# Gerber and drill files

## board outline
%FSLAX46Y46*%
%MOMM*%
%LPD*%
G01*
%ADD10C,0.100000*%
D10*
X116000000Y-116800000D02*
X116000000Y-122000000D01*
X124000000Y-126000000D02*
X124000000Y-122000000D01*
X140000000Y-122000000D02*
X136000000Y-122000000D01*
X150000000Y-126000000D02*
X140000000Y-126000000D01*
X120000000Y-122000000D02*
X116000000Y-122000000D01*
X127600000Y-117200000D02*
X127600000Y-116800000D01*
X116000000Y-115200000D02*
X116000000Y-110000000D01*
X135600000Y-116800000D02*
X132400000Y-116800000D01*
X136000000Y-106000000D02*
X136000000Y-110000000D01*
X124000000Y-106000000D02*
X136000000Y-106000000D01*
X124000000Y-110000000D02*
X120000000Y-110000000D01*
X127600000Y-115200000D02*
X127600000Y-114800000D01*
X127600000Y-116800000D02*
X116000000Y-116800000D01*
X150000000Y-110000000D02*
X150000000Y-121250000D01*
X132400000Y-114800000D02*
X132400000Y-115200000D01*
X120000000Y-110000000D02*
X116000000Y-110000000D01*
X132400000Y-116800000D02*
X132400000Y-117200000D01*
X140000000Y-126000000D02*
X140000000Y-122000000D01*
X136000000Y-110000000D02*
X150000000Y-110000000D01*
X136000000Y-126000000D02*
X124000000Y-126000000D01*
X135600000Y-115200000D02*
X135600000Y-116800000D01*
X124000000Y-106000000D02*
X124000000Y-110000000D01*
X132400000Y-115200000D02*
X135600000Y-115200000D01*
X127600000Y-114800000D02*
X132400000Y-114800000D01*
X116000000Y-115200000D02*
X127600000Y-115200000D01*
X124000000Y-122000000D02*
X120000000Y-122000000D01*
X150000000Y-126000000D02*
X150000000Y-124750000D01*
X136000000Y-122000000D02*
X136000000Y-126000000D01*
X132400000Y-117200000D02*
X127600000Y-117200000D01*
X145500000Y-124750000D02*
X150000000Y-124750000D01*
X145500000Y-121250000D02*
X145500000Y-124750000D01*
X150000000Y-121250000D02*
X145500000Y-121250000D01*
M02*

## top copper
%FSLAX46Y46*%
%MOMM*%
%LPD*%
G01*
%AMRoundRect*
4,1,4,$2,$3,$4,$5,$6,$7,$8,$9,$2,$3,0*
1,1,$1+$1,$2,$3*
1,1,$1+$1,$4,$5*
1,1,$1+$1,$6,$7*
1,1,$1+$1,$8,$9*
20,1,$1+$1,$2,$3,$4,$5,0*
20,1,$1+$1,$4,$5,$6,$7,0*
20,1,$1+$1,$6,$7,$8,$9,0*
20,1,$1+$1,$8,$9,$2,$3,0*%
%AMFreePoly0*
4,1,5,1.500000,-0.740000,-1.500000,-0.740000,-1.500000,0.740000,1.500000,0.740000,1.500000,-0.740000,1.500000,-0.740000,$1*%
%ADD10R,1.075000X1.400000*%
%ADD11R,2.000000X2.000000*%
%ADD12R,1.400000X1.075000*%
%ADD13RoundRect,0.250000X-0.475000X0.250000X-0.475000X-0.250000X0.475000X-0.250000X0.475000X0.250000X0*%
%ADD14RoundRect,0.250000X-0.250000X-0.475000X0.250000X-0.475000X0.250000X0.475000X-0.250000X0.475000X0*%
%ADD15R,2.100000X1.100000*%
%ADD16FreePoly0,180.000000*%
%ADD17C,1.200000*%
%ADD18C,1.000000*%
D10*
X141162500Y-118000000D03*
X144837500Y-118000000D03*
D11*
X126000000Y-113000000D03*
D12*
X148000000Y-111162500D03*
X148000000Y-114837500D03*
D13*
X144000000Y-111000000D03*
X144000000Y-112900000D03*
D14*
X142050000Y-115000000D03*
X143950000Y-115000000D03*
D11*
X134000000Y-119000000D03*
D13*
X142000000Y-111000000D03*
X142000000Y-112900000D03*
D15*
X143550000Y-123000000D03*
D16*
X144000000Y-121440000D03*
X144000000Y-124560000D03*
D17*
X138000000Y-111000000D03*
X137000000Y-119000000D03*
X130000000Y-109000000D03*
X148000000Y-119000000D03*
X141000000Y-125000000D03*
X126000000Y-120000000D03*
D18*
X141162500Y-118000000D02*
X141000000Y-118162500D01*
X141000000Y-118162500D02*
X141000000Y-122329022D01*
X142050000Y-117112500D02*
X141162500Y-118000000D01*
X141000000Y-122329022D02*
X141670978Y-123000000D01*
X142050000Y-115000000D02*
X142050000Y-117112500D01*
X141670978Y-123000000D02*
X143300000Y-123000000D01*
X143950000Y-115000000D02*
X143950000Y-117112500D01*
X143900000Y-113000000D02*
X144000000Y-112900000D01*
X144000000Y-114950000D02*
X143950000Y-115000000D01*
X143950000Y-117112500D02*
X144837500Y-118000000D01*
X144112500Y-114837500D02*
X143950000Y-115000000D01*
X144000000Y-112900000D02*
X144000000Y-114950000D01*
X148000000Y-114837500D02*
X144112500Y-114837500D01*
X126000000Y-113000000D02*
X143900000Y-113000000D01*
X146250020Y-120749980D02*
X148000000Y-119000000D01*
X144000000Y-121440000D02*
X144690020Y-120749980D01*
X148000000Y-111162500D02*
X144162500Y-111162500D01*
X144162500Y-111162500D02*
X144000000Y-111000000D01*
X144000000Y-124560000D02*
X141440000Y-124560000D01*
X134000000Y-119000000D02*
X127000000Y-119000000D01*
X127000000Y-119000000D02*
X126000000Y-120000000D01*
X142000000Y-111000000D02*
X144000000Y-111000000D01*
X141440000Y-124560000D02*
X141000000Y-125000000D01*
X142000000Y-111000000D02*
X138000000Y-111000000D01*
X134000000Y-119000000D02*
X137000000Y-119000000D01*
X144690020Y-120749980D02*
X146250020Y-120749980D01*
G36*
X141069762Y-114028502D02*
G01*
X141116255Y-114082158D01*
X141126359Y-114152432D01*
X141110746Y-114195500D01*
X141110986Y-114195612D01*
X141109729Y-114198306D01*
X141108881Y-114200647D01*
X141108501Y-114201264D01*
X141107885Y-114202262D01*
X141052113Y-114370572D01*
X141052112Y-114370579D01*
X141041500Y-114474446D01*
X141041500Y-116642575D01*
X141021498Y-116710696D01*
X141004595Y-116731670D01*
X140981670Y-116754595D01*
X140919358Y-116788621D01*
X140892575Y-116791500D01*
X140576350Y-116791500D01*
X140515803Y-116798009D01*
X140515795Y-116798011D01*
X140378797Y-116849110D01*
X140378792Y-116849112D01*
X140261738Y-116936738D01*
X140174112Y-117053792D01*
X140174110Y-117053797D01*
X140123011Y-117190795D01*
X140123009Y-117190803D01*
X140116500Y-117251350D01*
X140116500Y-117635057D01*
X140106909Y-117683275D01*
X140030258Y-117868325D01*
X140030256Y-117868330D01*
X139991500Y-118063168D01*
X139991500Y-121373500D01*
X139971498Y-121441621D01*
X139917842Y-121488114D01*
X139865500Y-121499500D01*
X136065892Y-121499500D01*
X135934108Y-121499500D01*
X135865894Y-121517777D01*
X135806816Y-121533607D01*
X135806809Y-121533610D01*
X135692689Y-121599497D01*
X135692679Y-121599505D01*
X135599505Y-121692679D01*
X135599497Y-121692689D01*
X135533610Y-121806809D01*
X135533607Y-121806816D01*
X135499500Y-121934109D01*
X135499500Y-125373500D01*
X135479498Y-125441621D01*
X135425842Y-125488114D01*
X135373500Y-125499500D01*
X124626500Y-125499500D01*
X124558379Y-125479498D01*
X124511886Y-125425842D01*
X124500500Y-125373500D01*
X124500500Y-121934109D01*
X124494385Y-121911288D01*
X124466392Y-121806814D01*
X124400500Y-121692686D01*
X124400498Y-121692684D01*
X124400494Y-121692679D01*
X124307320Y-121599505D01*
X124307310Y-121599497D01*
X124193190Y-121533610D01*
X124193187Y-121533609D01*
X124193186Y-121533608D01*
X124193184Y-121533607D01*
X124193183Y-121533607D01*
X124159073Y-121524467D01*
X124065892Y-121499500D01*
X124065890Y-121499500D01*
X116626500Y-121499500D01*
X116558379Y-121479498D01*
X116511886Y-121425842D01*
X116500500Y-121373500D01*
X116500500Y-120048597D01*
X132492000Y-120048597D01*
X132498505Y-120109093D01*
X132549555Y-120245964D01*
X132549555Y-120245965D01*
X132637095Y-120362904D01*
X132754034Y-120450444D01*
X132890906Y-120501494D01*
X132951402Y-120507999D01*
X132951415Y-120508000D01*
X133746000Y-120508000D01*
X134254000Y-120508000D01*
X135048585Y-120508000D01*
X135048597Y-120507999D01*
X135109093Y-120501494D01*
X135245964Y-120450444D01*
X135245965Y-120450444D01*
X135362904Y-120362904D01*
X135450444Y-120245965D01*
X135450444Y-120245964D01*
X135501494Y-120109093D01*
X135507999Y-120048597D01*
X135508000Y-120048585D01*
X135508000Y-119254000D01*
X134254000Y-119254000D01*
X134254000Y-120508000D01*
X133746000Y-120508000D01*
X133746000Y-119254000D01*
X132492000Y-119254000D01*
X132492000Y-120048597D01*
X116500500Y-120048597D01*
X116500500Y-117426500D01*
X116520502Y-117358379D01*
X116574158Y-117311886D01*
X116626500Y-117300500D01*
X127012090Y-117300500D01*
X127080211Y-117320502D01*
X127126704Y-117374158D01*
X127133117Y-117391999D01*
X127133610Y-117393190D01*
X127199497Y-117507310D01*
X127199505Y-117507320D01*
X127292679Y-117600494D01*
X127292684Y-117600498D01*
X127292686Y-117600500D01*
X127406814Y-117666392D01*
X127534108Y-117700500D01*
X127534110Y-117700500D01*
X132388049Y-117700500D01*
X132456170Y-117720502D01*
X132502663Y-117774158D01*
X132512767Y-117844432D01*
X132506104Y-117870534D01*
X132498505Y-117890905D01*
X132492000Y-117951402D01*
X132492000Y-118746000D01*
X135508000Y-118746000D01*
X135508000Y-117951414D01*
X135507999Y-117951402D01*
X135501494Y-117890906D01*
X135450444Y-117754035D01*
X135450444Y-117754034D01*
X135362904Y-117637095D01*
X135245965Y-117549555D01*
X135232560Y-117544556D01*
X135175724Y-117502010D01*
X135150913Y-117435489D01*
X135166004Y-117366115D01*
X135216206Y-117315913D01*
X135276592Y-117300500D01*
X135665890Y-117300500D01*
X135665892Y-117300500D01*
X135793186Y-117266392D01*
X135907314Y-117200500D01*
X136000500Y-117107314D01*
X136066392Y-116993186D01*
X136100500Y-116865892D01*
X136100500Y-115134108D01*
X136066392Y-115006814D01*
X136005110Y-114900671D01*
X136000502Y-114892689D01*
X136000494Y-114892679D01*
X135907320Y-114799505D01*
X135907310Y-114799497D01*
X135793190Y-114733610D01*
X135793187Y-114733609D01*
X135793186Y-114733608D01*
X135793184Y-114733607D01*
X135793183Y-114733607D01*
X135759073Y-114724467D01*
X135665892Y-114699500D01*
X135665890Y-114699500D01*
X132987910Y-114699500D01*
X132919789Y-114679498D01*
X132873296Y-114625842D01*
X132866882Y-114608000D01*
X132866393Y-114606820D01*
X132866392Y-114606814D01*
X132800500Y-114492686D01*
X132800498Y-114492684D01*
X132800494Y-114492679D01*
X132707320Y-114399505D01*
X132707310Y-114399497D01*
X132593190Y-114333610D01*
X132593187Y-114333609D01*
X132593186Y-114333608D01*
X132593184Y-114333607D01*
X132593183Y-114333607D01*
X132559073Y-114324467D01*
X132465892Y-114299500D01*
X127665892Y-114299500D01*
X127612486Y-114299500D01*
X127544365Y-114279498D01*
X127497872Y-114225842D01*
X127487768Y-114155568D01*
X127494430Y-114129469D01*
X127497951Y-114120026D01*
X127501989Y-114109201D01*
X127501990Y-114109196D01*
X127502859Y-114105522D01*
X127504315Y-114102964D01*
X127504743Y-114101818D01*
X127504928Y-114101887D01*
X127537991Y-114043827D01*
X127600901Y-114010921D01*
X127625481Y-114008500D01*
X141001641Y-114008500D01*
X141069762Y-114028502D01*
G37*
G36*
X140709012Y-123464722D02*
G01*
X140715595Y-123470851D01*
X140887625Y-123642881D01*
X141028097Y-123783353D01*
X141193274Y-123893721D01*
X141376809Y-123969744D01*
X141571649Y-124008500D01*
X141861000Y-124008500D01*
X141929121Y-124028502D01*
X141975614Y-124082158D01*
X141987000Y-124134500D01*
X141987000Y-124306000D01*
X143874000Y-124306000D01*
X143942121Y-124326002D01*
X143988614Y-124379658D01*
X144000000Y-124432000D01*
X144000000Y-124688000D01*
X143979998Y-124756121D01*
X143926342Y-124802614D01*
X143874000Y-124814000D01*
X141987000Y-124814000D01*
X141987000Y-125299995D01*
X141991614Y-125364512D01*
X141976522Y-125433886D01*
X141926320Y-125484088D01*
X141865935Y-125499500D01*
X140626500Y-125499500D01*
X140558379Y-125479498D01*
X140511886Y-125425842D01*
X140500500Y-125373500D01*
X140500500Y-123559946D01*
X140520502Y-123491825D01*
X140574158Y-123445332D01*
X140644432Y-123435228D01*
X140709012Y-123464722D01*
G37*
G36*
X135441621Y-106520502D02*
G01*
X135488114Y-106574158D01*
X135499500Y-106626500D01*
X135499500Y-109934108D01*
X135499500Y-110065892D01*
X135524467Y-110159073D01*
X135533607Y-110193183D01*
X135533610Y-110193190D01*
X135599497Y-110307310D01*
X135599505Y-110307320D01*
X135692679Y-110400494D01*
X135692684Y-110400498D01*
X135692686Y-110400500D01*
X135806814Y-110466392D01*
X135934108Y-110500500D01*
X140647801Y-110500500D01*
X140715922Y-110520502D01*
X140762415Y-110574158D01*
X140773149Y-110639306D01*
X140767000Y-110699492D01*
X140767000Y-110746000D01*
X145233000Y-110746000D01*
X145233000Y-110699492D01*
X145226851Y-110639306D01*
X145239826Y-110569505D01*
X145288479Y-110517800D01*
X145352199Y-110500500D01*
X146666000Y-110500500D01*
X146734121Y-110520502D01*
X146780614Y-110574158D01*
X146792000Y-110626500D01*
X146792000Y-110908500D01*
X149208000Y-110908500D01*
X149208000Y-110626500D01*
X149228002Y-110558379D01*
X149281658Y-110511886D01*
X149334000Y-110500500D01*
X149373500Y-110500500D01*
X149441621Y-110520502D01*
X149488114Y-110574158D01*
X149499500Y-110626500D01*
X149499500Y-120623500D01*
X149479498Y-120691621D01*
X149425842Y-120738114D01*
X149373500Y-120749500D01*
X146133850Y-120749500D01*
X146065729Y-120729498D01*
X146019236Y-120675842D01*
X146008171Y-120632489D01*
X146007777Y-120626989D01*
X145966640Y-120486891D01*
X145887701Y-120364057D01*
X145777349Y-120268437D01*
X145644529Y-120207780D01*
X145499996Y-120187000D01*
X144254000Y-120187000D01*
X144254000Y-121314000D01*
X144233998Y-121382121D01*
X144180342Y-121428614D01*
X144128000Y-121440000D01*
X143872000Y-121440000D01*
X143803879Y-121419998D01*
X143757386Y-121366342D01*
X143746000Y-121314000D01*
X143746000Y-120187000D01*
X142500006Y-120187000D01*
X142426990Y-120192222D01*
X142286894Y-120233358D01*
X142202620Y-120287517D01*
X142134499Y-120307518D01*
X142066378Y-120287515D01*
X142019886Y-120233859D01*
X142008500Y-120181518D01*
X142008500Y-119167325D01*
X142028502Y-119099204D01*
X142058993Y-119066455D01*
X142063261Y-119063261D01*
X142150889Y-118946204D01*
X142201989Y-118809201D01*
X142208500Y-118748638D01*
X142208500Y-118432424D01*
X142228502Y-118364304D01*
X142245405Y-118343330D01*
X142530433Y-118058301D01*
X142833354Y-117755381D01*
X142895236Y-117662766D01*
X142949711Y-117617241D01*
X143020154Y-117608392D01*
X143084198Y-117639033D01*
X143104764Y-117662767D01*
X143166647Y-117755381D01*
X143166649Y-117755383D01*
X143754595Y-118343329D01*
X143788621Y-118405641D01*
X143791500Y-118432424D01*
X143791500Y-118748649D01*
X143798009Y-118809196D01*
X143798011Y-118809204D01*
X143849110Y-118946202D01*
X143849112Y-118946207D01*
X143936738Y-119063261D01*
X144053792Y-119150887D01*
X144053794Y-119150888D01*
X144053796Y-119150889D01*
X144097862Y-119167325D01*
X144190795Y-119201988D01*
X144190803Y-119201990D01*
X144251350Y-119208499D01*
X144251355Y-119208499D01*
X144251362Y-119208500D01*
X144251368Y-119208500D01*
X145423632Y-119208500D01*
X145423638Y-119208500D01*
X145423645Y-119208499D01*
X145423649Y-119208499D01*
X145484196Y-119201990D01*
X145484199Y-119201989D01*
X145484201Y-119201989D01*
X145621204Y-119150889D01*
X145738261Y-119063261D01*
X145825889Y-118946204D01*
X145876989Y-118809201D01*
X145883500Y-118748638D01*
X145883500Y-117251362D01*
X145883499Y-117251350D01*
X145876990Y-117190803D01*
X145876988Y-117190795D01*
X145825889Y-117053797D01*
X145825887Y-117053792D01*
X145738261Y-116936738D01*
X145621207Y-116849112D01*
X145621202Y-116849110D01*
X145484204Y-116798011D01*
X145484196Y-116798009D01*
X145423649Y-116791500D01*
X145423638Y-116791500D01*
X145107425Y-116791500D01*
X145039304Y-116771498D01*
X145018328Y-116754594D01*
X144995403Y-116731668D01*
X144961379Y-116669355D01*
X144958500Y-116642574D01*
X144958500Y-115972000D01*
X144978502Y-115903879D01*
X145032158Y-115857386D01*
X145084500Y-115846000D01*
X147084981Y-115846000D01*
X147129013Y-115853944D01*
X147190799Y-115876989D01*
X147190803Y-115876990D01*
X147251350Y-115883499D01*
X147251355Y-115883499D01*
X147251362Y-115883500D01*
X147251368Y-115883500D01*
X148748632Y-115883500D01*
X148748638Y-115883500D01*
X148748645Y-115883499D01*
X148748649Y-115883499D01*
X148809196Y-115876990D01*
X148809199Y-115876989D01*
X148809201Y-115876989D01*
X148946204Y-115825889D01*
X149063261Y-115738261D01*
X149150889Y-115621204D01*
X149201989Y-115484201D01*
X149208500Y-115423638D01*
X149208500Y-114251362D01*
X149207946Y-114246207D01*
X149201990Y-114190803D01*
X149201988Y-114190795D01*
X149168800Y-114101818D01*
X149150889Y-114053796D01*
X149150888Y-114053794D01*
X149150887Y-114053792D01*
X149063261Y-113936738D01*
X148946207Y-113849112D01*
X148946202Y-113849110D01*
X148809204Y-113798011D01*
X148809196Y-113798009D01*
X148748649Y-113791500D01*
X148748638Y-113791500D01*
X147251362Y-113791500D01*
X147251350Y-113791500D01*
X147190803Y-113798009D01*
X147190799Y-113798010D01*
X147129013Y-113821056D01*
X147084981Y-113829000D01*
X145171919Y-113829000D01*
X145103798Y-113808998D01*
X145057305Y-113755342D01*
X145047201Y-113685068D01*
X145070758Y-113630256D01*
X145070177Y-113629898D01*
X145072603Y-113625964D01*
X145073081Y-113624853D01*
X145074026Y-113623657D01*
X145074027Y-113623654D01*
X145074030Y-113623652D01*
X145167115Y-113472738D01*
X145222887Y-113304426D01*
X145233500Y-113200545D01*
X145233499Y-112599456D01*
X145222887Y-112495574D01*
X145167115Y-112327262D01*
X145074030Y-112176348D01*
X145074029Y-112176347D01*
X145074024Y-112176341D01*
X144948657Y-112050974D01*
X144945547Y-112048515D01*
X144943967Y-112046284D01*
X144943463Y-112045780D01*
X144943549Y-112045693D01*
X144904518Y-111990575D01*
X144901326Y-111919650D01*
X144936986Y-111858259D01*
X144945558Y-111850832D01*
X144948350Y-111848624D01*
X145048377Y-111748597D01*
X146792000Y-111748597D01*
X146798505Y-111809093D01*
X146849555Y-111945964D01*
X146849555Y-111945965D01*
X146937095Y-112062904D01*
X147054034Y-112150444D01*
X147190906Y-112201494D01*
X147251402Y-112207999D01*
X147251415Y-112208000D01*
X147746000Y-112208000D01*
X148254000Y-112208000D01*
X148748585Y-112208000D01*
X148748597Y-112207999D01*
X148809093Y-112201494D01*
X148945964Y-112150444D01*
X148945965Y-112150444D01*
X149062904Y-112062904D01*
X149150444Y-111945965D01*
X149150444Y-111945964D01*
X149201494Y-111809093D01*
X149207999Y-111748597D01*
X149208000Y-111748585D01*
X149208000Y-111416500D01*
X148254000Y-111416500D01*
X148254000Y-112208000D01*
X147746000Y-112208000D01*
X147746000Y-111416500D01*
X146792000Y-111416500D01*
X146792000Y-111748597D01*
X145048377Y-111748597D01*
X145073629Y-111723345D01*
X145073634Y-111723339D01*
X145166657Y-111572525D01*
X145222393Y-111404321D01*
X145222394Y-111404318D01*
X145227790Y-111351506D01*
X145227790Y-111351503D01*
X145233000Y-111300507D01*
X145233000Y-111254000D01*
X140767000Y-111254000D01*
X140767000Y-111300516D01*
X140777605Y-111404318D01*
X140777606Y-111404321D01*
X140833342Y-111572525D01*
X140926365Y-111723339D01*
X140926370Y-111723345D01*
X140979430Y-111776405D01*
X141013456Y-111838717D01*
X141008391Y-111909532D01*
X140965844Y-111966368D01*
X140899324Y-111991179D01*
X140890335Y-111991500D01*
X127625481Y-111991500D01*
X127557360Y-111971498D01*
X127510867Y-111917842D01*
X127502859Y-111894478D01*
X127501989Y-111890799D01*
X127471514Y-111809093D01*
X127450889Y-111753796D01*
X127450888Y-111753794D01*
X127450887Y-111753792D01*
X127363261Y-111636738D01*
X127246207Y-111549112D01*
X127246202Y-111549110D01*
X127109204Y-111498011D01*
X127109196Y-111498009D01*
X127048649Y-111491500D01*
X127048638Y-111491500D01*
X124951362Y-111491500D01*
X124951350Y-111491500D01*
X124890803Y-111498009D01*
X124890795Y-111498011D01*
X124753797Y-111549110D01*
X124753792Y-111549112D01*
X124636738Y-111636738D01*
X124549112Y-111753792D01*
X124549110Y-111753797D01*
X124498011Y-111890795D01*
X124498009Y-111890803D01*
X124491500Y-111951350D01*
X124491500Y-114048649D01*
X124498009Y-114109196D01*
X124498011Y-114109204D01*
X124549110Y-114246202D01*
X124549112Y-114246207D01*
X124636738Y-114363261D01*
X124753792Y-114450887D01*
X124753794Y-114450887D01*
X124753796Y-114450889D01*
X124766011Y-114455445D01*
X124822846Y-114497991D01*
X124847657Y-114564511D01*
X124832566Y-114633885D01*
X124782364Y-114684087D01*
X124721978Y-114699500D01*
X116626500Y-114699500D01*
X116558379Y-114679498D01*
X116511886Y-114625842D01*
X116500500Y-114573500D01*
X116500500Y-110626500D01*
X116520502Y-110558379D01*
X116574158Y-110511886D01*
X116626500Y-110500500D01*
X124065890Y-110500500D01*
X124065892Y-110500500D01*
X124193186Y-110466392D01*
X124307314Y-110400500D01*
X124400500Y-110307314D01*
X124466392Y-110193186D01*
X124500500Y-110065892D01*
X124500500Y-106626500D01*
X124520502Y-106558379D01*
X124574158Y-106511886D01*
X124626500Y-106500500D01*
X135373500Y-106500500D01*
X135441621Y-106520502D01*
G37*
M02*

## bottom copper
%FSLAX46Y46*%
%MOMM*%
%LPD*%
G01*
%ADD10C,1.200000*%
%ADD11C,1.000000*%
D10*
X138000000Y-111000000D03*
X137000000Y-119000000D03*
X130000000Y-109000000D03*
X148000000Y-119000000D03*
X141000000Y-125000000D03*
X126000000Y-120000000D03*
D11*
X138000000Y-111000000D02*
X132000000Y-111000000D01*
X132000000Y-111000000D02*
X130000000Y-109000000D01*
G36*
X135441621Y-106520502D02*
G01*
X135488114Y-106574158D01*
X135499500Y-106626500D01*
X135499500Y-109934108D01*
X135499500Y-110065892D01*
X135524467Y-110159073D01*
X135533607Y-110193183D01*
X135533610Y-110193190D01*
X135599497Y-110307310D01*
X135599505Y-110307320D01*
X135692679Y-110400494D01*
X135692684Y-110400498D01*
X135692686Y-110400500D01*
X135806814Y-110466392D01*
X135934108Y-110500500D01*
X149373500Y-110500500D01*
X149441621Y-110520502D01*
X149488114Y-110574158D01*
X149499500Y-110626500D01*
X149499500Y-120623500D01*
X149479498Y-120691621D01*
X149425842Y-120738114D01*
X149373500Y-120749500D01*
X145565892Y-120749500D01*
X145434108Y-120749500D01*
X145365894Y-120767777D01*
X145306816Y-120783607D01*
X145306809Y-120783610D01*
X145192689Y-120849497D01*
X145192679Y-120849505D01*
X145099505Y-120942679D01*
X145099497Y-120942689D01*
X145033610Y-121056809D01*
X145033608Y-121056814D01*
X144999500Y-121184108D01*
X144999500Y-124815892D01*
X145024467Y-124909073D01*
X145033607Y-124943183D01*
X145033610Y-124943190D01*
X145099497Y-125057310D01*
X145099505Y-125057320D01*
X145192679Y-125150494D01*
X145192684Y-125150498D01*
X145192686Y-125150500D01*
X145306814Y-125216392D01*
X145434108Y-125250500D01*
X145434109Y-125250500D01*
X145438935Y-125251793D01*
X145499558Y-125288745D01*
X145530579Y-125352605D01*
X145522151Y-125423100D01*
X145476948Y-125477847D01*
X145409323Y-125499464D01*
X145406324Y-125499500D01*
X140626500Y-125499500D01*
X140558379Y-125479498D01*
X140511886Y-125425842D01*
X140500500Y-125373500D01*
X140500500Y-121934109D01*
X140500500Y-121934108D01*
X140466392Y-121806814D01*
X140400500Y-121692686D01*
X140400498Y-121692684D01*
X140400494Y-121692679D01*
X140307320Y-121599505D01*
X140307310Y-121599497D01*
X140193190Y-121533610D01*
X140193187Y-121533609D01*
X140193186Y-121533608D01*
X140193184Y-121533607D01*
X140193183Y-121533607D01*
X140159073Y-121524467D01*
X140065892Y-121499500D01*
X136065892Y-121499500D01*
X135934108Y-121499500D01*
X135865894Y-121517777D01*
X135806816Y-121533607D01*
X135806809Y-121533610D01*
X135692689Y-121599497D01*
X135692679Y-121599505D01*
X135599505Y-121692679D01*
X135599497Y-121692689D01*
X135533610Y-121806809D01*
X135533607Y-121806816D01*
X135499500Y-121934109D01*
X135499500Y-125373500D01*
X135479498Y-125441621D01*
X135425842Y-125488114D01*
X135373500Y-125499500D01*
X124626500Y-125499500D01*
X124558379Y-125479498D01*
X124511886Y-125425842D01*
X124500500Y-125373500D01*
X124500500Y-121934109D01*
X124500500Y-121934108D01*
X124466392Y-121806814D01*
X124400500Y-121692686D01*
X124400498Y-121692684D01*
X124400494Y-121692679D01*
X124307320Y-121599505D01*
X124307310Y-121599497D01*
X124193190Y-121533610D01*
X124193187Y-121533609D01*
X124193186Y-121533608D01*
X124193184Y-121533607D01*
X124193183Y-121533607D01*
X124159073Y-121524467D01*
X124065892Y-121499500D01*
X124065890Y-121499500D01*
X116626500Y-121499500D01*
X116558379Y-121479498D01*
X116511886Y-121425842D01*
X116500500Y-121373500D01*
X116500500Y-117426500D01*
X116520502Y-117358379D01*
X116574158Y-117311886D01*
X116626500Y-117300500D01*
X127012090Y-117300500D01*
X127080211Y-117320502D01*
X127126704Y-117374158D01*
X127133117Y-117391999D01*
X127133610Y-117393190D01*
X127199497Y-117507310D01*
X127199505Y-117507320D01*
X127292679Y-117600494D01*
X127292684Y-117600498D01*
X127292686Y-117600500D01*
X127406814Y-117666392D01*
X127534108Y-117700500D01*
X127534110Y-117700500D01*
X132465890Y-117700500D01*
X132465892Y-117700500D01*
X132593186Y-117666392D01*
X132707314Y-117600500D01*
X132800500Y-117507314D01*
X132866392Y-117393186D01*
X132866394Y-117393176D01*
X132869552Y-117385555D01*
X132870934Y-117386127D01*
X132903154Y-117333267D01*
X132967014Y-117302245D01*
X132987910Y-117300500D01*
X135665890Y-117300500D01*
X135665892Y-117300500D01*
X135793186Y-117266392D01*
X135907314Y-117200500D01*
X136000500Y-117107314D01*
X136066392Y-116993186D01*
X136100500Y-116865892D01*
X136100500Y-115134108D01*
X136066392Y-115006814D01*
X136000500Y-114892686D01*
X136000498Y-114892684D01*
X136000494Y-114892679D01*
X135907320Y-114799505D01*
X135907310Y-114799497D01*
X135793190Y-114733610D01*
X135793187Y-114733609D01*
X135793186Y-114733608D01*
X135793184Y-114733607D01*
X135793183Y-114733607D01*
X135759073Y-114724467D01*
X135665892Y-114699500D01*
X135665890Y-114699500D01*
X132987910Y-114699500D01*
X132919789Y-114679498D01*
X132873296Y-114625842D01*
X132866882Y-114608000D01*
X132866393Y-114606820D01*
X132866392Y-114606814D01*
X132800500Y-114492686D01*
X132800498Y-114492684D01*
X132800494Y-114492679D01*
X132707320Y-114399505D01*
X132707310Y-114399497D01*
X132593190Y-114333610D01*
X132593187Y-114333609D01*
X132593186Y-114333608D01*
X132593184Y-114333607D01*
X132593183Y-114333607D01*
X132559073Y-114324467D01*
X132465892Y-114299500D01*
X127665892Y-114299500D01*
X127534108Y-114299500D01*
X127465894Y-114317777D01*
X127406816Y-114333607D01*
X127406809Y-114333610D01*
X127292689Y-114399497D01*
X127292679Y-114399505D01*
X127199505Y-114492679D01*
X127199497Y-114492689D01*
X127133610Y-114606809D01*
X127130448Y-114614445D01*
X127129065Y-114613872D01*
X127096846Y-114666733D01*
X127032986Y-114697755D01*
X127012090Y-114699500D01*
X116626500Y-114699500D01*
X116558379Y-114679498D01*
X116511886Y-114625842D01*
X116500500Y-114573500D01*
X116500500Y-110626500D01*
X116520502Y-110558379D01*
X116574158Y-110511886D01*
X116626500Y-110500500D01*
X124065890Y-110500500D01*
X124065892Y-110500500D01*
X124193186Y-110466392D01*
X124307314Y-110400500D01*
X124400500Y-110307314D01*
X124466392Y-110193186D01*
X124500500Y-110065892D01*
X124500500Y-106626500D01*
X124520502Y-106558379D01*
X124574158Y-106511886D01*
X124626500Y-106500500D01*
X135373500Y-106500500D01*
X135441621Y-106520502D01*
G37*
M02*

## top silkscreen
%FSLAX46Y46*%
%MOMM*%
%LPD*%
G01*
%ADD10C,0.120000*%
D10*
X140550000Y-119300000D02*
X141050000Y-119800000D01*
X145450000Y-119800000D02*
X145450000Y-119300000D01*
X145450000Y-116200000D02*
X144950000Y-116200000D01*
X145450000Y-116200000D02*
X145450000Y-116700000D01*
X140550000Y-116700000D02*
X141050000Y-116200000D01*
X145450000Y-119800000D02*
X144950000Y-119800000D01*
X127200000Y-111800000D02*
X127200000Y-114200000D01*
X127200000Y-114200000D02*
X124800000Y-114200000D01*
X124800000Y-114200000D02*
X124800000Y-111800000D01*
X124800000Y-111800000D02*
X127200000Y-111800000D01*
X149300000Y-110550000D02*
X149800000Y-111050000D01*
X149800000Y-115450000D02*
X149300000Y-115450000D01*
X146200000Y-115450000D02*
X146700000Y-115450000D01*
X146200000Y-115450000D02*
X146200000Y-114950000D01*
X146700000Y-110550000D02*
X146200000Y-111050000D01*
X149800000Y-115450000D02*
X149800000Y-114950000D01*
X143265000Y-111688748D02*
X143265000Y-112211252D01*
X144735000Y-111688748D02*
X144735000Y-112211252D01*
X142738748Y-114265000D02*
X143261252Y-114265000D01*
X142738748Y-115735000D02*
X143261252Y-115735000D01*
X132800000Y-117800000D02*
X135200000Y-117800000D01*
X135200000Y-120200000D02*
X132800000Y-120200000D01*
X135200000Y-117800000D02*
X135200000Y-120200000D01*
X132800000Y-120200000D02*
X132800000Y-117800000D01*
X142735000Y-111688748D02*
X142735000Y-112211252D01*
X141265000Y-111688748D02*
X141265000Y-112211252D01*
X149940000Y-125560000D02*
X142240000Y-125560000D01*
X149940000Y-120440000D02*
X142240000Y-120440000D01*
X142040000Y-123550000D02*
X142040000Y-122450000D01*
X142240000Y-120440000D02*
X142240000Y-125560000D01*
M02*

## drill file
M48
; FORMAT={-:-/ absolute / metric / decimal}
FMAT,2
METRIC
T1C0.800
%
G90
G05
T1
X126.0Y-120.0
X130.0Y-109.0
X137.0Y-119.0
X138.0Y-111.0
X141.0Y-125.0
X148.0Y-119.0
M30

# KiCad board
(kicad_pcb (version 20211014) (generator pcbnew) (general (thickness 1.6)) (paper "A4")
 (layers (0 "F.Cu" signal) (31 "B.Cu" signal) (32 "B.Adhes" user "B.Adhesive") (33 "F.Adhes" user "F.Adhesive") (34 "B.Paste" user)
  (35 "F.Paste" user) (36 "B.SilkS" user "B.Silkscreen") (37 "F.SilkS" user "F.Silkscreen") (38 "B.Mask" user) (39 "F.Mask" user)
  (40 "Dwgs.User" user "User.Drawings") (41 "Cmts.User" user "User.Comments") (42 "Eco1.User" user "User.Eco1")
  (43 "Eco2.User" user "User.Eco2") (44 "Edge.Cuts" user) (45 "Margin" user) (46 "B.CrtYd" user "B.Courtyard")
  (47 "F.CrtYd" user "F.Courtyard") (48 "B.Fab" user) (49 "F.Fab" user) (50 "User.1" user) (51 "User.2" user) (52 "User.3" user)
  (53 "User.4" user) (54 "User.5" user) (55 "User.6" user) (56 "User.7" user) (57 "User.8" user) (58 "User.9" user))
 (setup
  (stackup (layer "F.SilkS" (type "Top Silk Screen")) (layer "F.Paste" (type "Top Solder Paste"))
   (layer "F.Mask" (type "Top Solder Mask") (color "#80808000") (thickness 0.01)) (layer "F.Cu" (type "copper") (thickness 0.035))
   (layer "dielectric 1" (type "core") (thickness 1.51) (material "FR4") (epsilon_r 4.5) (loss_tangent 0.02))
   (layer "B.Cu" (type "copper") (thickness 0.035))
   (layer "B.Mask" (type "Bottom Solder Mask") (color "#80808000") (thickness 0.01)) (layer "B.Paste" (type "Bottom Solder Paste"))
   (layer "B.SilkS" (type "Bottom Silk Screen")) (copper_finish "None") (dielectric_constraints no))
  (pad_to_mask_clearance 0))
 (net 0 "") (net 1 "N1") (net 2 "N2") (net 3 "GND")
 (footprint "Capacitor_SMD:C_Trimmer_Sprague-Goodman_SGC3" (layer "F.Cu") (at 143 118)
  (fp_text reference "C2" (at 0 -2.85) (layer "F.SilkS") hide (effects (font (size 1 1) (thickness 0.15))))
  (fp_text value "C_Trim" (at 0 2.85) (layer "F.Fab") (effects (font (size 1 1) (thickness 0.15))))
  (fp_line (start -2.45 1.3) (end -1.95 1.8) (layer "F.SilkS") (width 0.12))
  (fp_line (start 2.45 1.8) (end 2.45 1.3) (layer "F.SilkS") (width 0.12))
  (fp_line (start 2.45 -1.8) (end 1.95 -1.8) (layer "F.SilkS") (width 0.12))
  (fp_line (start 2.45 -1.8) (end 2.45 -1.3) (layer "F.SilkS") (width 0.12))
  (fp_line (start -2.45 -1.3) (end -1.95 -1.8) (layer "F.SilkS") (width 0.12))
  (fp_line (start 2.45 1.8) (end 1.95 1.8) (layer "F.SilkS") (width 0.12))
  (pad "1" smd rect locked (at -1.8375 0) (size 1.075 1.4) (layers "F.Cu" "F.Paste" "F.Mask") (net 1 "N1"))
  (pad "2" smd rect locked (at 1.8375 0) (size 1.075 1.4) (layers "F.Cu" "F.Paste" "F.Mask") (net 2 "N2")))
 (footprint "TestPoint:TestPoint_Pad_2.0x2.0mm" (layer "F.Cu") (at 126 113)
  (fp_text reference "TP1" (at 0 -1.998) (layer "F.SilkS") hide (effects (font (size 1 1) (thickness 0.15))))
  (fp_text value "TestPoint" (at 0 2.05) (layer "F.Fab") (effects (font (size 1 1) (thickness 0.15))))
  (fp_line (start 1.2 -1.2) (end 1.2 1.2) (layer "F.SilkS") (width 0.12))
  (fp_line (start 1.2 1.2) (end -1.2 1.2) (layer "F.SilkS") (width 0.12))
  (fp_line (start -1.2 1.2) (end -1.2 -1.2) (layer "F.SilkS") (width 0.12))
  (fp_line (start -1.2 -1.2) (end 1.2 -1.2) (layer "F.SilkS") (width 0.12))
  (pad "1" smd rect locked (at 0 0) (size 2 2) (layers "F.Cu" "F.Mask") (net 2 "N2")))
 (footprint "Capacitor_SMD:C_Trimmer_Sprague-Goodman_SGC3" (layer "F.Cu") (at 148 113 -90)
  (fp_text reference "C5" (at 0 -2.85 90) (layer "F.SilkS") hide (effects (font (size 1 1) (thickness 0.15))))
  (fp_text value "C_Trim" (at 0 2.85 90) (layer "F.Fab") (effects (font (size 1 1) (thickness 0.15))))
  (fp_line (start -2.45 -1.3) (end -1.95 -1.8) (layer "F.SilkS") (width 0.12))
  (fp_line (start 2.45 -1.8) (end 2.45 -1.3) (layer "F.SilkS") (width 0.12))
  (fp_line (start 2.45 1.8) (end 2.45 1.3) (layer "F.SilkS") (width 0.12))
  (fp_line (start 2.45 1.8) (end 1.95 1.8) (layer "F.SilkS") (width 0.12))
  (fp_line (start -2.45 1.3) (end -1.95 1.8) (layer "F.SilkS") (width 0.12))
  (fp_line (start 2.45 -1.8) (end 1.95 -1.8) (layer "F.SilkS") (width 0.12))
  (pad "1" smd rect locked (at -1.8375 0 270) (size 1.075 1.4) (layers "F.Cu" "F.Paste" "F.Mask") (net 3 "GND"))
  (pad "2" smd rect locked (at 1.8375 0 270) (size 1.075 1.4) (layers "F.Cu" "F.Paste" "F.Mask") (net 2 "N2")))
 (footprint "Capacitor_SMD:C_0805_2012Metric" (layer "F.Cu") (at 144 111.95 -90)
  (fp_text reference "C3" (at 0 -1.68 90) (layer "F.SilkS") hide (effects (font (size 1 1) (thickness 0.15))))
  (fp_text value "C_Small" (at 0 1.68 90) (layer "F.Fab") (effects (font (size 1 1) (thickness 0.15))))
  (fp_line (start -0.261252 0.735) (end 0.261252 0.735) (layer "F.SilkS") (width 0.12))
  (fp_line (start -0.261252 -0.735) (end 0.261252 -0.735) (layer "F.SilkS") (width 0.12))
  (pad "1" smd roundrect locked (at -0.95 0 270) (size 1 1.45) (layers "F.Cu" "F.Paste" "F.Mask") (roundrect_rratio 0.25) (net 3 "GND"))
  (pad "2" smd roundrect locked (at 0.95 0 270) (size 1 1.45) (layers "F.Cu" "F.Paste" "F.Mask") (roundrect_rratio 0.25) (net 2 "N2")))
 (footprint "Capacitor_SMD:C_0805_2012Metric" (layer "F.Cu") (at 143 115)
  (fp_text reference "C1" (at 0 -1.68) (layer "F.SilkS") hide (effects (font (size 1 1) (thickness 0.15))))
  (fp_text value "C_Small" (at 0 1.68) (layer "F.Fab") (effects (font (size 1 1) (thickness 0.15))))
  (fp_line (start -0.261252 -0.735) (end 0.261252 -0.735) (layer "F.SilkS") (width 0.12))
  (fp_line (start -0.261252 0.735) (end 0.261252 0.735) (layer "F.SilkS") (width 0.12))
  (pad "1" smd roundrect locked (at -0.95 0) (size 1 1.45) (layers "F.Cu" "F.Paste" "F.Mask") (roundrect_rratio 0.25) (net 1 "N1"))
  (pad "2" smd roundrect locked (at 0.95 0) (size 1 1.45) (layers "F.Cu" "F.Paste" "F.Mask") (roundrect_rratio 0.25) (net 2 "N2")))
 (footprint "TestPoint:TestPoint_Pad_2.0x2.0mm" (layer "F.Cu") (at 134 119)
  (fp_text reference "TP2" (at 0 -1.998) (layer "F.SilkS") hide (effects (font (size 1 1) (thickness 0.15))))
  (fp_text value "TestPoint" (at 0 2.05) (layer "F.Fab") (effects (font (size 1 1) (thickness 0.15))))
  (fp_line (start -1.2 -1.2) (end 1.2 -1.2) (layer "F.SilkS") (width 0.12))
  (fp_line (start 1.2 1.2) (end -1.2 1.2) (layer "F.SilkS") (width 0.12))
  (fp_line (start 1.2 -1.2) (end 1.2 1.2) (layer "F.SilkS") (width 0.12))
  (fp_line (start -1.2 1.2) (end -1.2 -1.2) (layer "F.SilkS") (width 0.12))
  (pad "1" smd rect locked (at 0 0) (size 2 2) (layers "F.Cu" "F.Mask") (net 3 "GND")))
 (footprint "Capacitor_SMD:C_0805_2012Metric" (layer "F.Cu") (at 142 111.95 -90)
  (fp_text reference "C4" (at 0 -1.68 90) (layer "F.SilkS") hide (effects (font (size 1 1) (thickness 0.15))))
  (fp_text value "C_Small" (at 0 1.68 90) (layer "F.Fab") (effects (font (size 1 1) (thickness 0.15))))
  (fp_line (start -0.261252 -0.735) (end 0.261252 -0.735) (layer "F.SilkS") (width 0.12))
  (fp_line (start -0.261252 0.735) (end 0.261252 0.735) (layer "F.SilkS") (width 0.12))
  (pad "1" smd roundrect locked (at -0.95 0 270) (size 1 1.45) (layers "F.Cu" "F.Paste" "F.Mask") (roundrect_rratio 0.25) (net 3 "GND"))
  (pad "2" smd roundrect locked (at 0.95 0 270) (size 1 1.45) (layers "F.Cu" "F.Paste" "F.Mask") (roundrect_rratio 0.25) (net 2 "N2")))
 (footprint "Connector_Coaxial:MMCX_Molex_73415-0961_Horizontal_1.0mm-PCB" (layer "F.Cu") (at 146.25 123 180)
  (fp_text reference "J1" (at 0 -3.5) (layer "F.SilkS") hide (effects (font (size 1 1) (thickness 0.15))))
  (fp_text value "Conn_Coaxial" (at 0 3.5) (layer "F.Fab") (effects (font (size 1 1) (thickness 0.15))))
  (fp_line (start -3.69 -2.56) (end 4.01 -2.56) (layer "F.SilkS") (width 0.12))
  (fp_line (start -3.69 2.56) (end 4.01 2.56) (layer "F.SilkS") (width 0.12))
  (fp_line (start 4.21 -0.55) (end 4.21 0.55) (layer "F.SilkS") (width 0.12))
  (fp_line (start 4.01 2.56) (end 4.01 -2.56) (layer "F.SilkS") (width 0.12))
  (fp_line (start 0.75 -1.75) (end -3.75 -1.75) (layer "Edge.Cuts") (width 0.1))
  (fp_line (start 0.75 1.75) (end 0.75 -1.75) (layer "Edge.Cuts") (width 0.1))
  (fp_line (start -3.75 1.75) (end 0.75 1.75) (layer "Edge.Cuts") (width 0.1))
  (pad "1" smd rect locked (at 2.7 0 180) (size 2.1 1.1) (layers "F.Cu" "F.Paste" "F.Mask") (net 1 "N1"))
  (pad "2" smd custom locked (at 2.25 1.56 180) (size 3 1.48) (layers "F.Cu" "F.Paste" "F.Mask") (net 3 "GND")
   (options (clearance outline) (anchor rect)) (primitives))
  (pad "2" smd custom locked (at 2.25 -1.56 180) (size 3 1.48) (layers "F.Cu" "F.Paste" "F.Mask") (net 3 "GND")
   (options (clearance outline) (anchor rect)) (primitives)))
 (gr_line (start 116 116.8) (end 116 122) (layer "Edge.Cuts") (width 0.1))
 (gr_line (start 124 126) (end 124 122) (layer "Edge.Cuts") (width 0.1))
 (gr_line (start 140 122) (end 136 122) (layer "Edge.Cuts") (width 0.1))
 (gr_line (start 150 126) (end 140 126) (layer "Edge.Cuts") (width 0.1))
 (gr_line (start 120 122) (end 116 122) (layer "Edge.Cuts") (width 0.1))
 (gr_line (start 127.6 117.2) (end 127.6 116.8) (layer "Edge.Cuts") (width 0.1))
 (gr_line (start 116 115.2) (end 116 110) (layer "Edge.Cuts") (width 0.1))
 (gr_line (start 135.6 116.8) (end 132.4 116.8) (layer "Edge.Cuts") (width 0.1))
 (gr_line (start 136 106) (end 136 110) (layer "Edge.Cuts") (width 0.1))
 (gr_line (start 124 106) (end 136 106) (layer "Edge.Cuts") (width 0.1))
 (gr_line (start 124 110) (end 120 110) (layer "Edge.Cuts") (width 0.1))
 (gr_line (start 127.6 115.2) (end 127.6 114.8) (layer "Edge.Cuts") (width 0.1))
 (gr_line (start 127.6 116.8) (end 116 116.8) (layer "Edge.Cuts") (width 0.1))
 (gr_line (start 150 110) (end 150 121.25) (layer "Edge.Cuts") (width 0.1))
 (gr_line (start 132.4 114.8) (end 132.4 115.2) (layer "Edge.Cuts") (width 0.1))
 (gr_line (start 120 110) (end 116 110) (layer "Edge.Cuts") (width 0.1))
 (gr_line (start 132.4 116.8) (end 132.4 117.2) (layer "Edge.Cuts") (width 0.1))
 (gr_line (start 140 126) (end 140 122) (layer "Edge.Cuts") (width 0.1))
 (gr_line (start 136 110) (end 150 110) (layer "Edge.Cuts") (width 0.1))
 (gr_line (start 136 126) (end 124 126) (layer "Edge.Cuts") (width 0.1))
 (gr_line (start 135.6 115.2) (end 135.6 116.8) (layer "Edge.Cuts") (width 0.1))
 (gr_line (start 124 106) (end 124 110) (layer "Edge.Cuts") (width 0.1))
 (gr_line (start 132.4 115.2) (end 135.6 115.2) (layer "Edge.Cuts") (width 0.1))
 (gr_line (start 127.6 114.8) (end 132.4 114.8) (layer "Edge.Cuts") (width 0.1))
 (gr_line (start 116 115.2) (end 127.6 115.2) (layer "Edge.Cuts") (width 0.1))
 (gr_line (start 124 122) (end 120 122) (layer "Edge.Cuts") (width 0.1))
 (gr_line (start 150 126) (end 150 124.75) (layer "Edge.Cuts") (width 0.1))
 (gr_line (start 136 122) (end 136 126) (layer "Edge.Cuts") (width 0.1))
 (gr_line (start 132.4 117.2) (end 127.6 117.2) (layer "Edge.Cuts") (width 0.1))
 (segment (start 141.1625 118) (end 141 118.1625) (width 1) (layer "F.Cu") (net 1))
 (segment (start 141 118.1625) (end 141 122.329022) (width 1) (layer "F.Cu") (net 1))
 (segment (start 142.05 117.1125) (end 141.1625 118) (width 1) (layer "F.Cu") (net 1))
 (segment (start 141 122.329022) (end 141.670978 123) (width 1) (layer "F.Cu") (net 1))
 (segment (start 142.05 115) (end 142.05 117.1125) (width 1) (layer "F.Cu") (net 1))
 (segment (start 141.670978 123) (end 143.3 123) (width 1) (layer "F.Cu") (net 1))
 (segment (start 143.95 115) (end 143.95 117.1125) (width 1) (layer "F.Cu") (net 2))
 (segment (start 143.9 113) (end 144 112.9) (width 1) (layer "F.Cu") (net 2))
 (segment (start 144 114.95) (end 143.95 115) (width 1) (layer "F.Cu") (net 2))
 (segment (start 143.95 117.1125) (end 144.8375 118) (width 1) (layer "F.Cu") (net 2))
 (segment (start 144.1125 114.8375) (end 143.95 115) (width 1) (layer "F.Cu") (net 2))
 (segment (start 144 112.9) (end 144 114.95) (width 1) (layer "F.Cu") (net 2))
 (segment (start 148 114.8375) (end 144.1125 114.8375) (width 1) (layer "F.Cu") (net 2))
 (segment (start 126 113) (end 143.9 113) (width 1) (layer "F.Cu") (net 2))
 (segment (start 146.25002 120.74998) (end 148 119) (width 1) (layer "F.Cu") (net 3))
 (segment (start 144 121.44) (end 144.69002 120.74998) (width 1) (layer "F.Cu") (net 3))
 (segment (start 148 111.1625) (end 144.1625 111.1625) (width 1) (layer "F.Cu") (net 3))
 (segment (start 144.1625 111.1625) (end 144 111) (width 1) (layer "F.Cu") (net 3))
 (segment (start 144 124.56) (end 141.44 124.56) (width 1) (layer "F.Cu") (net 3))
 (segment (start 134 119) (end 127 119) (width 1) (layer "F.Cu") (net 3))
 (segment (start 127 119) (end 126 120) (width 1) (layer "F.Cu") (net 3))
 (segment (start 142 111) (end 144 111) (width 1) (layer "F.Cu") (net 3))
 (segment (start 141.44 124.56) (end 141 125) (width 1) (layer "F.Cu") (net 3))
 (segment (start 142 111) (end 138 111) (width 1) (layer "F.Cu") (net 3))
 (segment (start 134 119) (end 137 119) (width 1) (layer "F.Cu") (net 3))
 (segment (start 144.69002 120.74998) (end 146.25002 120.74998) (width 1) (layer "F.Cu") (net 3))
 (via (at 138 111) (size 1.2) (drill 0.8) (layers "F.Cu" "B.Cu") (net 3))
 (via (at 137 119) (size 1.2) (drill 0.8) (layers "F.Cu" "B.Cu") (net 3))
 (via (at 130 109) (size 1.2) (drill 0.8) (layers "F.Cu" "B.Cu") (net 3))
 (via (at 148 119) (size 1.2) (drill 0.8) (layers "F.Cu" "B.Cu") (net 3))
 (via (at 141 125) (size 1.2) (drill 0.8) (layers "F.Cu" "B.Cu") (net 3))
 (via (at 126 120) (size 1.2) (drill 0.8) (layers "F.Cu" "B.Cu") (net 3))
 (segment (start 138 111) (end 132 111) (width 1) (layer "B.Cu") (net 3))
 (segment (start 132 111) (end 130 109) (width 1) (layer "B.Cu") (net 3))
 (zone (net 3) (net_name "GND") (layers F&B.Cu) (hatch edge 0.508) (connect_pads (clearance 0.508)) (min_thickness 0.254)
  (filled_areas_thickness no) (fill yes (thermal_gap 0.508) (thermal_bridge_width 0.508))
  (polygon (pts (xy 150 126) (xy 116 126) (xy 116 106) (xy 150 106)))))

